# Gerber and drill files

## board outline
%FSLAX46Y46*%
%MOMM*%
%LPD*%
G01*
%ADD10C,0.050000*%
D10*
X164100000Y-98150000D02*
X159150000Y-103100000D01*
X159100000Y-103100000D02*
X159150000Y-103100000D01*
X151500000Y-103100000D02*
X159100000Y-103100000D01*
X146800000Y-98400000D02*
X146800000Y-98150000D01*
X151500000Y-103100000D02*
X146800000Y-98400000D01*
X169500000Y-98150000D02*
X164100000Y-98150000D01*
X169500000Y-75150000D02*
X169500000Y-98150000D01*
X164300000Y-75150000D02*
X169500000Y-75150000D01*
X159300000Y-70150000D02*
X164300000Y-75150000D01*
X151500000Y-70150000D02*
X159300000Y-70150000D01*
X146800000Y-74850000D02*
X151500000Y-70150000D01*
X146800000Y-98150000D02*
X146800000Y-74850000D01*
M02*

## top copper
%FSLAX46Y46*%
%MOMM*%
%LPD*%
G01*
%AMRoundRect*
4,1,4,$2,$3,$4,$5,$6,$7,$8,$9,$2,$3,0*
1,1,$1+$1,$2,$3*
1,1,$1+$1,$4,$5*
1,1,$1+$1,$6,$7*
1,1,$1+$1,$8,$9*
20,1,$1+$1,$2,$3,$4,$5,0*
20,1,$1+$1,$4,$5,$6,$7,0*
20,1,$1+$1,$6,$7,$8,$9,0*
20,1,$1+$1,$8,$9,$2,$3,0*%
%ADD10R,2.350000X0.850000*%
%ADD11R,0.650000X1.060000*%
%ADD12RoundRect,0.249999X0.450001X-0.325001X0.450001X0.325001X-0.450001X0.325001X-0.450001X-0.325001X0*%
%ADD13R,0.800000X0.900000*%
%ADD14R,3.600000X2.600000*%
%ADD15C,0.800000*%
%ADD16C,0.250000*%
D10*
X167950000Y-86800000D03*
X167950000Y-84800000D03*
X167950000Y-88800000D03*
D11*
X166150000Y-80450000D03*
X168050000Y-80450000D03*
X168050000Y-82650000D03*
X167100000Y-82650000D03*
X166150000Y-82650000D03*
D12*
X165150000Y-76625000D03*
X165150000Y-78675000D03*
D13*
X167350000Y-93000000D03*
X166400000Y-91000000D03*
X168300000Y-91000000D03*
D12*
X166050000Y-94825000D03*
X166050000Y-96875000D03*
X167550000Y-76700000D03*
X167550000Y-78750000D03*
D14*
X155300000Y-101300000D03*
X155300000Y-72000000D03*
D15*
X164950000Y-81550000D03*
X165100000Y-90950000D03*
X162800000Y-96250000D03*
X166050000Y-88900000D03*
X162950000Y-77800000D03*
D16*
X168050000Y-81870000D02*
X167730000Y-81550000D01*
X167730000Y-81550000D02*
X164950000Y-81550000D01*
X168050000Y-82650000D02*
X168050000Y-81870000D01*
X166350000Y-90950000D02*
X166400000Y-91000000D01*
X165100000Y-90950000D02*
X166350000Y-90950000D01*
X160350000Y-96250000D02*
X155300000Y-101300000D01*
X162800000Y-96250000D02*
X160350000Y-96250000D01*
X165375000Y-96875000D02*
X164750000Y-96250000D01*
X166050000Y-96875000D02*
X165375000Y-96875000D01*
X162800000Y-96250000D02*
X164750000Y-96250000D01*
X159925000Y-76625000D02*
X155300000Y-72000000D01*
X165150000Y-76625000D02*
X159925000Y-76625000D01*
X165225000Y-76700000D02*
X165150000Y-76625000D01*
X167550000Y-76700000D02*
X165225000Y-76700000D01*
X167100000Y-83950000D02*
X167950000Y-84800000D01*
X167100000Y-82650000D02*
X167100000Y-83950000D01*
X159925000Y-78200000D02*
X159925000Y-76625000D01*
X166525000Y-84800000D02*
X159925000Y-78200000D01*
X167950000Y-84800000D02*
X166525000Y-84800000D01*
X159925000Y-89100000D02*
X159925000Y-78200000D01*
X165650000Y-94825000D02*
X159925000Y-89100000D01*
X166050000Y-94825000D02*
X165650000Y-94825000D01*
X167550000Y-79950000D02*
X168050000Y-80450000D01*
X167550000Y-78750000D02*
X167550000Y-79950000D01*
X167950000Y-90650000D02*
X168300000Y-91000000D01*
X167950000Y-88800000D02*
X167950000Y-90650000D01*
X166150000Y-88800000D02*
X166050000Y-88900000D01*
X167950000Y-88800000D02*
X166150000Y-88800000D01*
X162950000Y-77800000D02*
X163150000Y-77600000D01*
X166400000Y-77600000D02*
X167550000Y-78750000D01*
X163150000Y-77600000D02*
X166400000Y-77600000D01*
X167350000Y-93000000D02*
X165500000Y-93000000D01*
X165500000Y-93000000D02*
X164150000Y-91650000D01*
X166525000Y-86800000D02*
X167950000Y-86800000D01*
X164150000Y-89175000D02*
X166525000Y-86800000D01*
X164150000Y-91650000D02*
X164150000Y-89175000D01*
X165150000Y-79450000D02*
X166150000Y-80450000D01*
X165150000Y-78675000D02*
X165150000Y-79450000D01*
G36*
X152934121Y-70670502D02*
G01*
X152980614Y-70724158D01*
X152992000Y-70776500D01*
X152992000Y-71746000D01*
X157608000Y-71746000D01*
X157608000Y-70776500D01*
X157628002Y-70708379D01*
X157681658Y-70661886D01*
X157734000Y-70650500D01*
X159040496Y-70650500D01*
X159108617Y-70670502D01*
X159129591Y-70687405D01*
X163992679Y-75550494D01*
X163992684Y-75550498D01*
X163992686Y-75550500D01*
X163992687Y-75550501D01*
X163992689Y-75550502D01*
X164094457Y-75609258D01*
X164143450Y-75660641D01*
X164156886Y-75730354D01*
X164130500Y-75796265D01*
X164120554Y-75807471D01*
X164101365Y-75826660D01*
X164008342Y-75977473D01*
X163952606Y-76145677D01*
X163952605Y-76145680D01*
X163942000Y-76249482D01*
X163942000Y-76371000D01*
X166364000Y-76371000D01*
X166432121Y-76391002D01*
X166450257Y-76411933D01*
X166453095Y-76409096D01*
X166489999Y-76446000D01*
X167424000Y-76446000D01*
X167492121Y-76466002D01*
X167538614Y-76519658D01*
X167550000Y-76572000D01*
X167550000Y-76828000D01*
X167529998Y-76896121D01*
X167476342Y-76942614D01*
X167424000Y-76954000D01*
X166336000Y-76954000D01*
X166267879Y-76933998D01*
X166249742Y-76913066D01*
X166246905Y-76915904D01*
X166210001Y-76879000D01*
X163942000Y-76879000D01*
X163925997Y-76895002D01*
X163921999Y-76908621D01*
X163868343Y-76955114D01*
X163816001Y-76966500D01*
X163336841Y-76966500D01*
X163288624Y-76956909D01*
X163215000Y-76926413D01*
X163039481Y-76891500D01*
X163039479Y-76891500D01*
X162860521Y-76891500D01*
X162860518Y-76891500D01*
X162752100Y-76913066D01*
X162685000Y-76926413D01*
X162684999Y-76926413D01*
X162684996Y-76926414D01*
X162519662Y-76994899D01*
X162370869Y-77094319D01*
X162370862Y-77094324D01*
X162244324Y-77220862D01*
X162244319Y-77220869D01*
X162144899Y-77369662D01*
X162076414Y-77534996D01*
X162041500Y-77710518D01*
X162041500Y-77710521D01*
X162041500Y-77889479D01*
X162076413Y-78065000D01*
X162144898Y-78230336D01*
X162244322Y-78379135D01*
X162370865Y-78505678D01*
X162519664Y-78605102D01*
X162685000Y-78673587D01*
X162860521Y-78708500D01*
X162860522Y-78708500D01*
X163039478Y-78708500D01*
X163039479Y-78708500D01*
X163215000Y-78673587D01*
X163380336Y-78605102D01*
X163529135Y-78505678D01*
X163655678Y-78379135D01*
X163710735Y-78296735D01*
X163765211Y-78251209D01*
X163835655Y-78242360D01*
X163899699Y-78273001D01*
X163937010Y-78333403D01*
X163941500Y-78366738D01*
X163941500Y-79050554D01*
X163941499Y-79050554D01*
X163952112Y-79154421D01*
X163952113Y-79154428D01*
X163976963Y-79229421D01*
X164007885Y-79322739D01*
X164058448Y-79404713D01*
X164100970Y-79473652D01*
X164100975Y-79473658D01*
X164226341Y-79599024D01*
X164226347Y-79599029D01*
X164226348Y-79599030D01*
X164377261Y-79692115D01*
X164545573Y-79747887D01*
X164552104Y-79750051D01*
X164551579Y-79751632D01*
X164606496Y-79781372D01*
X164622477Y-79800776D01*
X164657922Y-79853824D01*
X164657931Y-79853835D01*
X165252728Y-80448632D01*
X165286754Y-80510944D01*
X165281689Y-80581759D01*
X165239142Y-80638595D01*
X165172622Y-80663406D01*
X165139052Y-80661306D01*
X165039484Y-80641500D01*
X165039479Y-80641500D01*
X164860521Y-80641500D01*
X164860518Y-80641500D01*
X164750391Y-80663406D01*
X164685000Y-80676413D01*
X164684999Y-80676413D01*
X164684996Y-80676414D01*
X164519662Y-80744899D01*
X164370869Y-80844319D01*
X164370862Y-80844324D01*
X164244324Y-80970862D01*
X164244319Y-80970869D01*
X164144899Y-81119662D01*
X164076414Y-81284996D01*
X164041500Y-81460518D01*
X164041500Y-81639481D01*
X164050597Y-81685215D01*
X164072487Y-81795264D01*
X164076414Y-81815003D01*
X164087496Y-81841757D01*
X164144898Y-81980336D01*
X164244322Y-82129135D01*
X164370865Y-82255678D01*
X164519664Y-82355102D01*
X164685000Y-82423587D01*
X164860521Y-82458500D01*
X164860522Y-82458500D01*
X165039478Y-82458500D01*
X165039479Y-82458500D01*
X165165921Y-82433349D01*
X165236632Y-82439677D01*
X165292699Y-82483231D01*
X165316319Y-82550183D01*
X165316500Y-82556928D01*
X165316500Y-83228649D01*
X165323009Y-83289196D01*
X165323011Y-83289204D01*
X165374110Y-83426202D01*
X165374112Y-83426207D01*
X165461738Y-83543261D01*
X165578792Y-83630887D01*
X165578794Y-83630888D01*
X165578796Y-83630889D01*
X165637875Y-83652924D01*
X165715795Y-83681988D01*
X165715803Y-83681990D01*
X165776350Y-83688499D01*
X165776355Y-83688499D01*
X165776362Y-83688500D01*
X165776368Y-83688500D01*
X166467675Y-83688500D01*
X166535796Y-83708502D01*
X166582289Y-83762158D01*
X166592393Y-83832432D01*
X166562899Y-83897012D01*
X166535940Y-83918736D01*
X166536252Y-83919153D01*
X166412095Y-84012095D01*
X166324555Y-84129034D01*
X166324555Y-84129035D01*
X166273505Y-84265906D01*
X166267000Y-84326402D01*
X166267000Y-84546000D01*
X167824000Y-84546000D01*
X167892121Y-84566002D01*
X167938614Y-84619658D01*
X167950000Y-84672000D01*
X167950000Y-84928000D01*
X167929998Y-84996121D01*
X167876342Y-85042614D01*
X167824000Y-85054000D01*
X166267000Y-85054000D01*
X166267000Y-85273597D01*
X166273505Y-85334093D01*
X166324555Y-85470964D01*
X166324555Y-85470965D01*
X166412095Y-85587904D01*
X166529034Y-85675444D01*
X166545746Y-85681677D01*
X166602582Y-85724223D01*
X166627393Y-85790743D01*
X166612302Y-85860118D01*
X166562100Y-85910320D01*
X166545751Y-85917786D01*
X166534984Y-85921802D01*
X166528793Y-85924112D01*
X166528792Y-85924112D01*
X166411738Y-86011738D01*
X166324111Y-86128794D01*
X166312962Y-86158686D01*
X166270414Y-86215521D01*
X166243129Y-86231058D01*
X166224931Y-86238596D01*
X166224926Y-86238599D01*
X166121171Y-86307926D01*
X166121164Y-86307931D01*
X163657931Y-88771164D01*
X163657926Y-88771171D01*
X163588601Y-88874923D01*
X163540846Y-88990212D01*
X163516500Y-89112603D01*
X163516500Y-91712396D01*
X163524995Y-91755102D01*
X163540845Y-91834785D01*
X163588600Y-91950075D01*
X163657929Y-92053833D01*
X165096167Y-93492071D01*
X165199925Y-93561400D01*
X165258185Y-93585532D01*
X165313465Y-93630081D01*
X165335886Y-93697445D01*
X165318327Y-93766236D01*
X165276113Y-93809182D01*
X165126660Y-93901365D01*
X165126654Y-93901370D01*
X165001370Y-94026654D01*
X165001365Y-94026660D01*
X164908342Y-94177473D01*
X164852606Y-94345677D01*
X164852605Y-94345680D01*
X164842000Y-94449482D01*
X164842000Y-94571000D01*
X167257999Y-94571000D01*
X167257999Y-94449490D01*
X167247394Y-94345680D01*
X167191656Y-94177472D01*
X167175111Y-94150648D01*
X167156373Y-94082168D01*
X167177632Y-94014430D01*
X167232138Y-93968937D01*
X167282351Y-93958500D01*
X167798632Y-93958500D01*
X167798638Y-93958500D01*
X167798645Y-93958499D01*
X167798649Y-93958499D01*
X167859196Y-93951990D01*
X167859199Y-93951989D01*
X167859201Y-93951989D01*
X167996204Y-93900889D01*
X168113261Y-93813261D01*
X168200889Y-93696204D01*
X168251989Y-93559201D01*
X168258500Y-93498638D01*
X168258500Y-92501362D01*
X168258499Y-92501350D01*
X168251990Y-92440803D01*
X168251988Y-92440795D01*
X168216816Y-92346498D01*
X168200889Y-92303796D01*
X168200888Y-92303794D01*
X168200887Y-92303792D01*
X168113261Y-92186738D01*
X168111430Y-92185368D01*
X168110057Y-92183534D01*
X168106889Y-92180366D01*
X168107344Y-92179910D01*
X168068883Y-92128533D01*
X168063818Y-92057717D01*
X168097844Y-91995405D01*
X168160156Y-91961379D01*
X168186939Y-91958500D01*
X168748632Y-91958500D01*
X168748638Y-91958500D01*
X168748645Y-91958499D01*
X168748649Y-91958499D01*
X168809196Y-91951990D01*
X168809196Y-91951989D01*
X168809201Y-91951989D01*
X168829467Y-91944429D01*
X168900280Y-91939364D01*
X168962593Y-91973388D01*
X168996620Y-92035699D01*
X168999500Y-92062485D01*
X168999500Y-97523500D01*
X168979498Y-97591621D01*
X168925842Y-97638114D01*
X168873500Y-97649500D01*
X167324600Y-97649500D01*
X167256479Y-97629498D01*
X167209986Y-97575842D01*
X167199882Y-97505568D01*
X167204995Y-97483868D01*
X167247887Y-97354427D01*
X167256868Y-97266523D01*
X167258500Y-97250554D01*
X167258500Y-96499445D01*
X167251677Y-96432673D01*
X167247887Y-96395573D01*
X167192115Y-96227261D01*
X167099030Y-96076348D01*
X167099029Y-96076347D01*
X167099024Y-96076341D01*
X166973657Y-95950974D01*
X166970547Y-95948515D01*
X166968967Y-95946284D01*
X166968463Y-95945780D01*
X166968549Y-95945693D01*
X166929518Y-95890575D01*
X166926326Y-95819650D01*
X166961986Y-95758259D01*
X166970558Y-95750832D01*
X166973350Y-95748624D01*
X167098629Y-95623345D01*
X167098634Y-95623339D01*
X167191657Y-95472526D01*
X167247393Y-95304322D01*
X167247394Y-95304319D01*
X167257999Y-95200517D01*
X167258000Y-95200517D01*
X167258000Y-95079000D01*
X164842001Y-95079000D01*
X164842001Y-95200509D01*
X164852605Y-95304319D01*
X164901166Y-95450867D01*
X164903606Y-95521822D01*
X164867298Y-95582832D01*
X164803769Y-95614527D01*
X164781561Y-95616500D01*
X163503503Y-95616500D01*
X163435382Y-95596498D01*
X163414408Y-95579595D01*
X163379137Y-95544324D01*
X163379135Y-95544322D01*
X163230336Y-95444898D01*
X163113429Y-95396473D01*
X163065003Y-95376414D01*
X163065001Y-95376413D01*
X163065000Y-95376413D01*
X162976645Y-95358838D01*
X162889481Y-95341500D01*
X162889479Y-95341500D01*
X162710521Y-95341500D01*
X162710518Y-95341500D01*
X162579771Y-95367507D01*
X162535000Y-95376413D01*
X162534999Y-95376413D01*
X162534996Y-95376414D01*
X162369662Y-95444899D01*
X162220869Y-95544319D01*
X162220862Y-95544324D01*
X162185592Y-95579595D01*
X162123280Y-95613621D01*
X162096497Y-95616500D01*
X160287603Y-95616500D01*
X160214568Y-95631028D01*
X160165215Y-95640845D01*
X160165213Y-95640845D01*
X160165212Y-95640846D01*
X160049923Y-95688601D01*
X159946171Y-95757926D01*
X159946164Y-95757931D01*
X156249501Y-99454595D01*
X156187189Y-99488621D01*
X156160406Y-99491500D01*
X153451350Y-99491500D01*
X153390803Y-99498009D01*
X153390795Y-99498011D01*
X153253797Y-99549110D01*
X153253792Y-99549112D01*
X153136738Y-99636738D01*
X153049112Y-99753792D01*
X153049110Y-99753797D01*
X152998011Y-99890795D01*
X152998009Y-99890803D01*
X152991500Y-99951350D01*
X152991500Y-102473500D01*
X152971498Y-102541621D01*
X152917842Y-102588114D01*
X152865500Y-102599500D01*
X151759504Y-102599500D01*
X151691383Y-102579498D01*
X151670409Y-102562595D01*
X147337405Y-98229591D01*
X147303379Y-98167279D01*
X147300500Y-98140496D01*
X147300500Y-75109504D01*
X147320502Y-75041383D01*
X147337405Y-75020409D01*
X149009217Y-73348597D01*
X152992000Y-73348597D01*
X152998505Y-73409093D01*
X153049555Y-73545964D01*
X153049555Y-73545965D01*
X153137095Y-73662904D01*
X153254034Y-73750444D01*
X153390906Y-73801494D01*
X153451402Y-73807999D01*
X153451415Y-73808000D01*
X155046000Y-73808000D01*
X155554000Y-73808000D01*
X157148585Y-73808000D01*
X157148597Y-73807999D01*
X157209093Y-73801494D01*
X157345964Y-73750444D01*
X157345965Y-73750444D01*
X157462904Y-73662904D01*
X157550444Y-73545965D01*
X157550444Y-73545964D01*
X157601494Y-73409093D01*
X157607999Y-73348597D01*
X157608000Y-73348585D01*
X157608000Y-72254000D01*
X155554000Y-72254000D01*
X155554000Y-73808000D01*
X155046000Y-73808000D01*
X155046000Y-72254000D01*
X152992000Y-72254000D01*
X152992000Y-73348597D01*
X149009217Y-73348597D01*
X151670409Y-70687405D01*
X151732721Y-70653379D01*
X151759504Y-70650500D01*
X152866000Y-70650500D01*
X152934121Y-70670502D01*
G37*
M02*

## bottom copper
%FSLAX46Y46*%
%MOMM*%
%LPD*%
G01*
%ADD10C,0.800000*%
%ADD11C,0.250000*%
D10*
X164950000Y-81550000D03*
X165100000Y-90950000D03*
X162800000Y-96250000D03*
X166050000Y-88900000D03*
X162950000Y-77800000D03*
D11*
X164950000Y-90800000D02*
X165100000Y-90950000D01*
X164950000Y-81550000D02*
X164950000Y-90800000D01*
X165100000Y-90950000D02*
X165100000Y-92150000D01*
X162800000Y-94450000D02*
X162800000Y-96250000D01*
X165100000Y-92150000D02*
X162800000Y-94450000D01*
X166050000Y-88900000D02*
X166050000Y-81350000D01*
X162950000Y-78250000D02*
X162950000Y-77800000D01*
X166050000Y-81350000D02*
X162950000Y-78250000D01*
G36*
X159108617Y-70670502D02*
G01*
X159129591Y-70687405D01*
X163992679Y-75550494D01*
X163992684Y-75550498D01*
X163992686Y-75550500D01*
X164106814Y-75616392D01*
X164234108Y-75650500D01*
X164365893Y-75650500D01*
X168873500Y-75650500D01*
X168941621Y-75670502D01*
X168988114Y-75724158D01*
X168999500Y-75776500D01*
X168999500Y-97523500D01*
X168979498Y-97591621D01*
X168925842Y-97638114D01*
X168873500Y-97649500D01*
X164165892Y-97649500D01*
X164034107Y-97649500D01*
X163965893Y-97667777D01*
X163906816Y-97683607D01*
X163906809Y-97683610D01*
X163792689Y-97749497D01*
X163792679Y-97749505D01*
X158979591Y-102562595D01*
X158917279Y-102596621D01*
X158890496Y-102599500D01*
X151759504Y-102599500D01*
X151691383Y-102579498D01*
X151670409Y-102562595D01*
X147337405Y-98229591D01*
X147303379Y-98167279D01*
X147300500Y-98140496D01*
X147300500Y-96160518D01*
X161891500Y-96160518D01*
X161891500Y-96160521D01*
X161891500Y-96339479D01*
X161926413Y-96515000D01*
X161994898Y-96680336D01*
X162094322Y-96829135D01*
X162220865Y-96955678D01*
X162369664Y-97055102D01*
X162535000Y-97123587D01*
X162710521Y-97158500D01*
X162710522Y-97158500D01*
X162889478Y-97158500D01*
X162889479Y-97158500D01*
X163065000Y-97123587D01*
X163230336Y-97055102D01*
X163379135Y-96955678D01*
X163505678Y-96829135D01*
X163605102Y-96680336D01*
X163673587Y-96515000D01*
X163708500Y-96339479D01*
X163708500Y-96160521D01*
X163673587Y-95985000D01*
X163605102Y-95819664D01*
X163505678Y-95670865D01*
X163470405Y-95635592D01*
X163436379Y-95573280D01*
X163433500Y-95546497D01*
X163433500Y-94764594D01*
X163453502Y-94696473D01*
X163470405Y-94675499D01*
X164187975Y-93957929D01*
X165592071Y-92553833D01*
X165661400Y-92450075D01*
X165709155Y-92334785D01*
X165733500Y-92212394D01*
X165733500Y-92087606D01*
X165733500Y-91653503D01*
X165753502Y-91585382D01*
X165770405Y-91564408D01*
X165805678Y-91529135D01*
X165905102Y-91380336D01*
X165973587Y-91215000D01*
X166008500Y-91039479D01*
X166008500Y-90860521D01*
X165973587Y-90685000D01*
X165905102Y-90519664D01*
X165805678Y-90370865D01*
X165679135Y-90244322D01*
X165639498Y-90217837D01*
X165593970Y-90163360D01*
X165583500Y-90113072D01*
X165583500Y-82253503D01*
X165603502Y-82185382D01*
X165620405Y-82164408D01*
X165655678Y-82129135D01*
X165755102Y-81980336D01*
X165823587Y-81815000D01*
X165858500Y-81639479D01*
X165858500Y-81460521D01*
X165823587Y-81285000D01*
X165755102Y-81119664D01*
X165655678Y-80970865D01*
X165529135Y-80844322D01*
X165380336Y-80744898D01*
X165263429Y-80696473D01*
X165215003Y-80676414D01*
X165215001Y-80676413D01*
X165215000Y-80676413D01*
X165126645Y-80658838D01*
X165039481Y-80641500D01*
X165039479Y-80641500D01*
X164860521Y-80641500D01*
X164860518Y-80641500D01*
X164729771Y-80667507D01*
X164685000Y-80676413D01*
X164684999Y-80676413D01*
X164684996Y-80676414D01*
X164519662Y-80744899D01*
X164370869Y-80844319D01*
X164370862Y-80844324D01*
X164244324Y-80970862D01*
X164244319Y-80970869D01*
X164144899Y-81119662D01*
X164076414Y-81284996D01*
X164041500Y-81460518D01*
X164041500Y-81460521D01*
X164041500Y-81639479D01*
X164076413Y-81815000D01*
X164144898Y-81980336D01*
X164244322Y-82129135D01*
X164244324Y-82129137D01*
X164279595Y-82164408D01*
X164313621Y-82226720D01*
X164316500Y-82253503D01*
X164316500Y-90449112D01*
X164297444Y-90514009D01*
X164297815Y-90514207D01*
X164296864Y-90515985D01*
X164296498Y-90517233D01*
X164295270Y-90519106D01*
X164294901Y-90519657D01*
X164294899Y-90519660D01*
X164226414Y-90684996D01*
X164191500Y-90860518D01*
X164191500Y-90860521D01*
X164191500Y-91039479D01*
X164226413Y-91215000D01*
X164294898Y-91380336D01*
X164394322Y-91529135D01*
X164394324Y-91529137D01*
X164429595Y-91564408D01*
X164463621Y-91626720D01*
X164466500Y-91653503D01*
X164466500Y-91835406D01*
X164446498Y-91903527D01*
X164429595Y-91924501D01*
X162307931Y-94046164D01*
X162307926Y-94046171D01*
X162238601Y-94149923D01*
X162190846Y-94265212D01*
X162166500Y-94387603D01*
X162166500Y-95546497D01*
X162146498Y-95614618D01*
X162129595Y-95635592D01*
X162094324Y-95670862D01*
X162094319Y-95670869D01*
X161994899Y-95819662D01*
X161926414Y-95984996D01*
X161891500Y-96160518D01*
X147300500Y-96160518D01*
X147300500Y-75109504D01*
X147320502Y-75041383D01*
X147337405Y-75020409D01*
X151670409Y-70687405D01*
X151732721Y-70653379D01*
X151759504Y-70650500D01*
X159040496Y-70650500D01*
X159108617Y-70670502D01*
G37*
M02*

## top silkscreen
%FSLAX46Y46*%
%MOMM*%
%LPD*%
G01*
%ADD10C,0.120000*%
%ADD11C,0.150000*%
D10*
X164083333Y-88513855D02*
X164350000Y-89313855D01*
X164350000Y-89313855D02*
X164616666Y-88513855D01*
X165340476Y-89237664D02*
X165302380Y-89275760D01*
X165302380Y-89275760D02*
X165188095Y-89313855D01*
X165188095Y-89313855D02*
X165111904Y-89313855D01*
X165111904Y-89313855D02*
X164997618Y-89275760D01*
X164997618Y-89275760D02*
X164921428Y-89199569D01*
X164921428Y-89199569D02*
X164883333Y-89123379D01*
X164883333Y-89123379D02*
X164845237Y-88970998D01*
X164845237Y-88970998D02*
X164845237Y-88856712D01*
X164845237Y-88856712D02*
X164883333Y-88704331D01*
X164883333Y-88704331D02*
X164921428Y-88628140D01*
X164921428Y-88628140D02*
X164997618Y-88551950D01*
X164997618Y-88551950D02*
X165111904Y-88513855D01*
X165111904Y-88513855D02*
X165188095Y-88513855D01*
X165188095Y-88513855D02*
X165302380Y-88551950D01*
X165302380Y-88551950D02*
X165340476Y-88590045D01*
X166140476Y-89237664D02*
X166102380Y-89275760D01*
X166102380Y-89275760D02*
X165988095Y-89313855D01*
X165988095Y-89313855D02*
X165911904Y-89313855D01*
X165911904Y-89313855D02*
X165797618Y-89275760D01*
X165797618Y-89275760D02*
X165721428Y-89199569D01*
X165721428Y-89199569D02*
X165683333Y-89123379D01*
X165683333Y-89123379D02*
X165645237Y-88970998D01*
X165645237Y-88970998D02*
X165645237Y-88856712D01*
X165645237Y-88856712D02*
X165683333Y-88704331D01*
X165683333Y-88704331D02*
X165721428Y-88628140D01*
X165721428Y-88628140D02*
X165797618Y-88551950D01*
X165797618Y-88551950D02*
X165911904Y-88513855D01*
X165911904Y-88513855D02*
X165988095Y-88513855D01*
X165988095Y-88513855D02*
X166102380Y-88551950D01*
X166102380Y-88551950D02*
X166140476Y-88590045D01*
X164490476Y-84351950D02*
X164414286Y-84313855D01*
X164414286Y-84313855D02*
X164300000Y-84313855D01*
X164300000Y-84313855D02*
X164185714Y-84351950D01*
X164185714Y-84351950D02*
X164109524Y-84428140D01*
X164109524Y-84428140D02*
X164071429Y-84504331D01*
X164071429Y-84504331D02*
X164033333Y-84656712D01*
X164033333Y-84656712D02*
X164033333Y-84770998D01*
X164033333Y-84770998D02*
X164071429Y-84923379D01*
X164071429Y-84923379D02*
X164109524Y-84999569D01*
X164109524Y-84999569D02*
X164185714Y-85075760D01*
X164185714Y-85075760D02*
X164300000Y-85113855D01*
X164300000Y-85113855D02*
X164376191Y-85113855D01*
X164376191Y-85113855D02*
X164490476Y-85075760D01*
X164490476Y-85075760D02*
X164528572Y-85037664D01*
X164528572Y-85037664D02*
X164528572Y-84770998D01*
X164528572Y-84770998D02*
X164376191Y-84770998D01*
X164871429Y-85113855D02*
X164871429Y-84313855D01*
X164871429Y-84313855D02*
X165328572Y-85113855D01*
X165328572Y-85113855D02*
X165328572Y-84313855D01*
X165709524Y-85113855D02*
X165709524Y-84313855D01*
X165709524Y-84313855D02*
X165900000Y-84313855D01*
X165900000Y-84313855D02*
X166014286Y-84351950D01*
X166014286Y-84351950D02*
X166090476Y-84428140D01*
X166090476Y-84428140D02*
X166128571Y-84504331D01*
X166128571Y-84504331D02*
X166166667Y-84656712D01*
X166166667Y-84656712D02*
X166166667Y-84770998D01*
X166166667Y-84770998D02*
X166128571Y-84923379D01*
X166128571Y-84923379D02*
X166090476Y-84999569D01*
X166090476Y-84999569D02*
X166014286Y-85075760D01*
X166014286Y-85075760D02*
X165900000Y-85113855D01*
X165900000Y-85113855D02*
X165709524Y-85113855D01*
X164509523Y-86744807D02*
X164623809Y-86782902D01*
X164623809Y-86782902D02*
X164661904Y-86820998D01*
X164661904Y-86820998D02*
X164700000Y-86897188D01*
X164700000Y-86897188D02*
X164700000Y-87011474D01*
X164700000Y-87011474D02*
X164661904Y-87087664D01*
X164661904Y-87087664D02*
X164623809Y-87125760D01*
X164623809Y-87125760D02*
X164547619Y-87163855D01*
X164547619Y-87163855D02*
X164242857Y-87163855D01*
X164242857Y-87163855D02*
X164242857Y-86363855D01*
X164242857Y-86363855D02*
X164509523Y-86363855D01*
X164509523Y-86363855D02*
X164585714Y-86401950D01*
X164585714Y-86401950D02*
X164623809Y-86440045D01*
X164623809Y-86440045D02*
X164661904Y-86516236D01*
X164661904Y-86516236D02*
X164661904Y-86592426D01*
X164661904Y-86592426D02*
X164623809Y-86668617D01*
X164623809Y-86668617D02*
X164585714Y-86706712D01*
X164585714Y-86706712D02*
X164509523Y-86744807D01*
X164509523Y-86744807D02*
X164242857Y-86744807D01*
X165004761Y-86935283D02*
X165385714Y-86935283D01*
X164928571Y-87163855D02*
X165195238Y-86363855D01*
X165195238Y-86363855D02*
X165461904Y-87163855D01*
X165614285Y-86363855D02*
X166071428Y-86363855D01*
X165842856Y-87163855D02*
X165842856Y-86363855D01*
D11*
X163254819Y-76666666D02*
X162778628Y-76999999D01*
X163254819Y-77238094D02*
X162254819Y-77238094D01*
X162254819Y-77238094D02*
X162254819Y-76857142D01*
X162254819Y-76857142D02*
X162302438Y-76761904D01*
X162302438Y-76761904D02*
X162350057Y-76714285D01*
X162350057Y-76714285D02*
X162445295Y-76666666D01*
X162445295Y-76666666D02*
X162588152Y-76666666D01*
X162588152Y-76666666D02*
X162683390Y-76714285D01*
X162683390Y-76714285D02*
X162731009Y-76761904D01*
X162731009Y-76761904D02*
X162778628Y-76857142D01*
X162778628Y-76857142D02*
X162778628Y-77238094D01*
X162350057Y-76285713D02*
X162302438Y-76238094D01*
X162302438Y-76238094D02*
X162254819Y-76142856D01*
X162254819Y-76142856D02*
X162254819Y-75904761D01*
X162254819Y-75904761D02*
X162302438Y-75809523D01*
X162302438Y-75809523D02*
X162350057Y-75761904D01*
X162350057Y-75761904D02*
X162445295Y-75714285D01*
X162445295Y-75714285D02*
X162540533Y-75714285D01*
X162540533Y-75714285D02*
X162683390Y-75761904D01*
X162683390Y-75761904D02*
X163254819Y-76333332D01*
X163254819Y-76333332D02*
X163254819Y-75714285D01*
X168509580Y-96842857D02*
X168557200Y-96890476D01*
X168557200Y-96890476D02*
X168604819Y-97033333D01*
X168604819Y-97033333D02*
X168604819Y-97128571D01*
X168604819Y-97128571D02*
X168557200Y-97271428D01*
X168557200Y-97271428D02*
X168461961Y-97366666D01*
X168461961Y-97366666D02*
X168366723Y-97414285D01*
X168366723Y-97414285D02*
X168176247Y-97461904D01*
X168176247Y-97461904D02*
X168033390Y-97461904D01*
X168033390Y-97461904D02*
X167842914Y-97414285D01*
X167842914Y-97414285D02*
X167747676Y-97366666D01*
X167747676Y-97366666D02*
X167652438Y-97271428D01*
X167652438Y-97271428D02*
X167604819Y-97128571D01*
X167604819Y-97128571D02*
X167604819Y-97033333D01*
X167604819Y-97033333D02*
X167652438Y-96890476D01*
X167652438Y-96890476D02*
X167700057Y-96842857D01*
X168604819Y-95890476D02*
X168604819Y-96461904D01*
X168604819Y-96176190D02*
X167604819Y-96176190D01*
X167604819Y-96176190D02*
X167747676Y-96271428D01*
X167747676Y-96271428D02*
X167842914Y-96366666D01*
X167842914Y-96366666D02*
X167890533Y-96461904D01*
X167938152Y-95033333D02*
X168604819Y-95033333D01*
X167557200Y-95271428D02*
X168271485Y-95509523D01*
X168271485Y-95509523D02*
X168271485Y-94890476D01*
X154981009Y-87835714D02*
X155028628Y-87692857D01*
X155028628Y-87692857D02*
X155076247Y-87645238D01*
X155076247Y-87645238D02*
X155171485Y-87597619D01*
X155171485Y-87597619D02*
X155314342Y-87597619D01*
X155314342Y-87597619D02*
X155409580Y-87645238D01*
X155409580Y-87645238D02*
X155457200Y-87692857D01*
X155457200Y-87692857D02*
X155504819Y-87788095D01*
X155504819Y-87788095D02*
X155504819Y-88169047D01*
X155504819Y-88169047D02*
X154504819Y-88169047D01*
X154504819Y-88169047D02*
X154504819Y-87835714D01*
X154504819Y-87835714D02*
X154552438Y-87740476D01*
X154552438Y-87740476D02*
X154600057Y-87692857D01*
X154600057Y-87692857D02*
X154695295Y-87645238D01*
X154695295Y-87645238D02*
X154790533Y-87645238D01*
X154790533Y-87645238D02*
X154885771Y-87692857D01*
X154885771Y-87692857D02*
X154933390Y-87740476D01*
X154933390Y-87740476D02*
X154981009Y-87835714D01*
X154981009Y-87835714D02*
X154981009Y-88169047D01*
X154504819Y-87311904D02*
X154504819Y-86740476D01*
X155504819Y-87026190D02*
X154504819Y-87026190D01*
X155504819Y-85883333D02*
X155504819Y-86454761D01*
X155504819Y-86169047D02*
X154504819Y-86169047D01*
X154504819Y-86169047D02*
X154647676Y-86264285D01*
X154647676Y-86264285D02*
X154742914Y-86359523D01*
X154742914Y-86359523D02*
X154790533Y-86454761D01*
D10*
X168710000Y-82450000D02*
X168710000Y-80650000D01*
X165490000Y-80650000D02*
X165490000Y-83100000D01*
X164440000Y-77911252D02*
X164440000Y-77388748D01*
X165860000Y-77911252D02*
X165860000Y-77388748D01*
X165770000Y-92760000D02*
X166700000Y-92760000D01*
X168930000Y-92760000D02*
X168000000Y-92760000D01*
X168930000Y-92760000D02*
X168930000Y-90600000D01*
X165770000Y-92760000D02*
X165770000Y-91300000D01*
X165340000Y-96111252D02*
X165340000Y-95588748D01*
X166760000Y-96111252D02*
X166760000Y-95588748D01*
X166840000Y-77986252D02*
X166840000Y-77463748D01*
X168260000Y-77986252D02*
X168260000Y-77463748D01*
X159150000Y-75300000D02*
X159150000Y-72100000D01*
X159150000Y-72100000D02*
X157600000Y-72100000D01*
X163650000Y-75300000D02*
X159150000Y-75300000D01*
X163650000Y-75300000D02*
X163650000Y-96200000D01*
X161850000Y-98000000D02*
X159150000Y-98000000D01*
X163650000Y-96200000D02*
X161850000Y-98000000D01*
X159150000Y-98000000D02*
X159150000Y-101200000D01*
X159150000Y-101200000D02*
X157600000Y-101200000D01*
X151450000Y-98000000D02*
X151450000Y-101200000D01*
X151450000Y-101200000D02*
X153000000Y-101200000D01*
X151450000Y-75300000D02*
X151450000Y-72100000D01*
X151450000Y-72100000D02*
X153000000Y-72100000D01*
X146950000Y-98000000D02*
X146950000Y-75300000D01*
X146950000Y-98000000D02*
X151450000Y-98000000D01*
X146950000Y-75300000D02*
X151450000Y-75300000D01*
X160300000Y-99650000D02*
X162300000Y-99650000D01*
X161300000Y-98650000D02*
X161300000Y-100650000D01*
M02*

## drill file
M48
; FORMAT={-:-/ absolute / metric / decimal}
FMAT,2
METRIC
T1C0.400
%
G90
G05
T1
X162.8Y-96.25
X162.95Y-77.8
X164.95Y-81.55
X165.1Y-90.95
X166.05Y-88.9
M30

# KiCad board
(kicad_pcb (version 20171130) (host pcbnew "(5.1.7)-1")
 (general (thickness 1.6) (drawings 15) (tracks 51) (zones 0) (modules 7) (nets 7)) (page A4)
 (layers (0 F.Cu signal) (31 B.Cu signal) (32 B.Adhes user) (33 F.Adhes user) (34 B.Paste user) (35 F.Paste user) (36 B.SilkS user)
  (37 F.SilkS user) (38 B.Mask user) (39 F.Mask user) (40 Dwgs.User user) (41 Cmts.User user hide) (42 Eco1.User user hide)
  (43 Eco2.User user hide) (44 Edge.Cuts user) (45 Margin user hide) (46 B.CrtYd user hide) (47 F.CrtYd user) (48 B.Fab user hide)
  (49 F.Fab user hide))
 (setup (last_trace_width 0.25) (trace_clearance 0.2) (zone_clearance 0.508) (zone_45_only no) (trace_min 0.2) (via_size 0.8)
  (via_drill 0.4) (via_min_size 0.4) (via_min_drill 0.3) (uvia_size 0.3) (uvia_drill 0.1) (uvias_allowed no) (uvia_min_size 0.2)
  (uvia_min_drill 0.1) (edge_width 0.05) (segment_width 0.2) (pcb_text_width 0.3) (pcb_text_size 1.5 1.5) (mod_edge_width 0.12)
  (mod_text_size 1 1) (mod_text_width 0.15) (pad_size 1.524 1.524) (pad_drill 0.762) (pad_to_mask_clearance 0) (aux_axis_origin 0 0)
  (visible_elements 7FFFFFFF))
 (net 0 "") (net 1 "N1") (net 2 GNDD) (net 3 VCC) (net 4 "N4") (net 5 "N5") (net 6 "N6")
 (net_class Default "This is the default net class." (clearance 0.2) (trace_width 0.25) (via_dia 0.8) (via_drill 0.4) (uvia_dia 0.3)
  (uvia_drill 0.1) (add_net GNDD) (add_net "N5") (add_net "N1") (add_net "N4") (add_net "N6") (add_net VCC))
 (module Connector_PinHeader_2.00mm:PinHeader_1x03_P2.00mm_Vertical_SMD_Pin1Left (layer F.Cu) (at 167.95 86.8 180)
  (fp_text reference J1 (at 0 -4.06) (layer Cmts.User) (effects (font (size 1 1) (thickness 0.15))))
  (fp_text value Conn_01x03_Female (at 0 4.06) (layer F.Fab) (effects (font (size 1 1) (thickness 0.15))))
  (pad 2 smd rect (at 0 0 180) (size 2.35 0.85) (layers F.Cu F.Paste F.Mask) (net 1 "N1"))
  (pad 3 smd rect (at 0 2 180) (size 2.35 0.85) (layers F.Cu F.Paste F.Mask) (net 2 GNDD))
  (pad 1 smd rect (at 0 -2 180) (size 2.35 0.85) (layers F.Cu F.Paste F.Mask) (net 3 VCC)))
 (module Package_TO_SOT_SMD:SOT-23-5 (layer F.Cu) (at 167.1 81.55 90)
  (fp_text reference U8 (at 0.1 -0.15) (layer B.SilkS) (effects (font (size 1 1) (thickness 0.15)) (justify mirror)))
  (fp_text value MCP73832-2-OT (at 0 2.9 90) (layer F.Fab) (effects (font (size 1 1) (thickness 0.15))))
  (fp_line (start -0.9 1.61) (end 0.9 1.61) (layer F.SilkS) (width 0.12))
  (fp_line (start 0.9 -1.61) (end -1.55 -1.61) (layer F.SilkS) (width 0.12))
  (pad 5 smd rect (at 1.1 -0.95 90) (size 1.06 0.65) (layers F.Cu F.Paste F.Mask) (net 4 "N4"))
  (pad 4 smd rect (at 1.1 0.95 90) (size 1.06 0.65) (layers F.Cu F.Paste F.Mask) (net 3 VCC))
  (pad 3 smd rect (at -1.1 0.95 90) (size 1.06 0.65) (layers F.Cu F.Paste F.Mask) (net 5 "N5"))
  (pad 2 smd rect (at -1.1 0 90) (size 1.06 0.65) (layers F.Cu F.Paste F.Mask) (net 2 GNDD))
  (pad 1 smd rect (at -1.1 -0.95 90) (size 1.06 0.65) (layers F.Cu F.Paste F.Mask) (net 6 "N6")))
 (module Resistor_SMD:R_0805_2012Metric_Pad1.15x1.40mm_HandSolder (layer F.Cu) (at 165.15 77.65 90)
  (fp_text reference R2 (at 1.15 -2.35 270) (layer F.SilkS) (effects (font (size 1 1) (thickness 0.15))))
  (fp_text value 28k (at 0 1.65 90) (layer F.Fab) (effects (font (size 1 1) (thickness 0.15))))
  (fp_line (start -0.261252 -0.71) (end 0.261252 -0.71) (layer F.SilkS) (width 0.12))
  (fp_line (start -0.261252 0.71) (end 0.261252 0.71) (layer F.SilkS) (width 0.12))
  (pad 2 smd roundrect (at 1.025 0 90) (size 1.15 1.4) (layers F.Cu F.Paste F.Mask) (roundrect_rratio 0.2173904347826087) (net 2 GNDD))
  (pad 1 smd roundrect (at -1.025 0 90) (size 1.15 1.4) (layers F.Cu F.Paste F.Mask) (roundrect_rratio 0.2173904347826087) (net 4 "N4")))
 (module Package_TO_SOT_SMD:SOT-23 (layer F.Cu) (at 167.35 92 270)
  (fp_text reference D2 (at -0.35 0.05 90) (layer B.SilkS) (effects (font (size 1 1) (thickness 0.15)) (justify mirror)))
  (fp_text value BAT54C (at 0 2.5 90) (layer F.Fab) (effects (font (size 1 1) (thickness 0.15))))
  (fp_line (start 0.76 1.58) (end 0.76 0.65) (layer F.SilkS) (width 0.12))
  (fp_line (start 0.76 -1.58) (end 0.76 -0.65) (layer F.SilkS) (width 0.12))
  (fp_line (start 0.76 -1.58) (end -1.4 -1.58) (layer F.SilkS) (width 0.12))
  (fp_line (start 0.76 1.58) (end -0.7 1.58) (layer F.SilkS) (width 0.12))
  (pad 3 smd rect (at 1 0 270) (size 0.9 0.8) (layers F.Cu F.Paste F.Mask) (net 1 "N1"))
  (pad 2 smd rect (at -1 0.95 270) (size 0.9 0.8) (layers F.Cu F.Paste F.Mask) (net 5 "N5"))
  (pad 1 smd rect (at -1 -0.95 270) (size 0.9 0.8) (layers F.Cu F.Paste F.Mask) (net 3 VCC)))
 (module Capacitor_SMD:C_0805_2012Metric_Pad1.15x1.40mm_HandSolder (layer F.Cu) (at 166.05 95.85 90)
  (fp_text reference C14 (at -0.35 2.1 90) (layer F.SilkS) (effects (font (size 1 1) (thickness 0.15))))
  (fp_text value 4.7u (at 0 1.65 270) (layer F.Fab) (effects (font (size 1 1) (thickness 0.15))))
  (fp_line (start -0.261252 -0.71) (end 0.261252 -0.71) (layer F.SilkS) (width 0.12))
  (fp_line (start -0.261252 0.71) (end 0.261252 0.71) (layer F.SilkS) (width 0.12))
  (pad 2 smd roundrect (at 1.025 0 90) (size 1.15 1.4) (layers F.Cu F.Paste F.Mask) (roundrect_rratio 0.2173904347826087) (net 2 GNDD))
  (pad 1 smd roundrect (at -1.025 0 90) (size 1.15 1.4) (layers F.Cu F.Paste F.Mask) (roundrect_rratio 0.2173904347826087) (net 5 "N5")))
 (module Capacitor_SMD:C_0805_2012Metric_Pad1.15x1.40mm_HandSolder (layer F.Cu) (at 167.55 77.725 90)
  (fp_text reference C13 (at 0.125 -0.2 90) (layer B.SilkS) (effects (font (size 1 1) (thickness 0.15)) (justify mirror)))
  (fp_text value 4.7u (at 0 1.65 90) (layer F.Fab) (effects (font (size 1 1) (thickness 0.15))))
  (fp_line (start -0.261252 -0.71) (end 0.261252 -0.71) (layer F.SilkS) (width 0.12))
  (fp_line (start -0.261252 0.71) (end 0.261252 0.71) (layer F.SilkS) (width 0.12))
  (pad 2 smd roundrect (at 1.025 0 90) (size 1.15 1.4) (layers F.Cu F.Paste F.Mask) (roundrect_rratio 0.2173904347826087) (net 2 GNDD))
  (pad 1 smd roundrect (at -1.025 0 90) (size 1.15 1.4) (layers F.Cu F.Paste F.Mask) (roundrect_rratio 0.2173904347826087) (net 3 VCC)))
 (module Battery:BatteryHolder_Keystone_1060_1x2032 (layer F.Cu) (at 155.3 86.65 90)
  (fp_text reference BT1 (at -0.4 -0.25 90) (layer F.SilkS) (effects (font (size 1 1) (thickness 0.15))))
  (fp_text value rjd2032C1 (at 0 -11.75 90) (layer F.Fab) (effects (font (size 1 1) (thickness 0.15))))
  (fp_line (start 11.35 3.85) (end 14.55 3.85) (layer F.SilkS) (width 0.12))
  (fp_line (start 14.55 3.85) (end 14.55 2.3) (layer F.SilkS) (width 0.12))
  (fp_line (start 11.35 8.35) (end 11.35 3.85) (layer F.SilkS) (width 0.12))
  (fp_line (start 11.35 8.35) (end -9.55 8.35) (layer F.SilkS) (width 0.12))
  (fp_line (start -11.35 6.55) (end -11.35 3.85) (layer F.SilkS) (width 0.12))
  (fp_line (start -9.55 8.35) (end -11.35 6.55) (layer F.SilkS) (width 0.12))
  (fp_line (start -11.35 3.85) (end -14.55 3.85) (layer F.SilkS) (width 0.12))
  (fp_line (start -14.55 3.85) (end -14.55 2.3) (layer F.SilkS) (width 0.12))
  (fp_line (start -11.35 -3.85) (end -14.55 -3.85) (layer F.SilkS) (width 0.12))
  (fp_line (start -14.55 -3.85) (end -14.55 -2.3) (layer F.SilkS) (width 0.12))
  (fp_line (start 11.35 -3.85) (end 14.55 -3.85) (layer F.SilkS) (width 0.12))
  (fp_line (start 14.55 -3.85) (end 14.55 -2.3) (layer F.SilkS) (width 0.12))
  (fp_line (start -11.35 -8.35) (end 11.35 -8.35) (layer F.SilkS) (width 0.12))
  (fp_line (start -11.35 -8.35) (end -11.35 -3.85) (layer F.SilkS) (width 0.12))
  (fp_line (start 11.35 -8.35) (end 11.35 -3.85) (layer F.SilkS) (width 0.12))
  (fp_line (start -13 5) (end -13 7) (layer F.SilkS) (width 0.12))
  (fp_line (start -12 6) (end -14 6) (layer F.SilkS) (width 0.12))
  (pad 1 smd rect (at -14.65 0 270) (size 2.6 3.6) (layers F.Cu F.Paste F.Mask) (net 5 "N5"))
  (pad 2 smd rect (at 14.65 0 270) (size 2.6 3.6) (layers F.Cu F.Paste F.Mask) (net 2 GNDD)))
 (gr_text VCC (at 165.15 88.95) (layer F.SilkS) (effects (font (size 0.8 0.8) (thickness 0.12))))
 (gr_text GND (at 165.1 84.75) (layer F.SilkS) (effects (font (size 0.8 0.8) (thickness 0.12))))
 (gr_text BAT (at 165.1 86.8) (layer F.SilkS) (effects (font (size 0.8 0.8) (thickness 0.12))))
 (gr_line (start 164.1 98.15) (end 159.15 103.1) (layer Edge.Cuts) (width 0.05))
 (gr_line (start 159.1 103.1) (end 159.15 103.1) (layer Edge.Cuts) (width 0.05))
 (gr_line (start 151.5 103.1) (end 159.1 103.1) (layer Edge.Cuts) (width 0.05))
 (gr_line (start 146.8 98.4) (end 146.8 98.15) (layer Edge.Cuts) (width 0.05))
 (gr_line (start 151.5 103.1) (end 146.8 98.4) (layer Edge.Cuts) (width 0.05))
 (gr_line (start 169.5 98.15) (end 164.1 98.15) (layer Edge.Cuts) (width 0.05))
 (gr_line (start 169.5 75.15) (end 169.5 98.15) (layer Edge.Cuts) (width 0.05))
 (gr_line (start 164.3 75.15) (end 169.5 75.15) (layer Edge.Cuts) (width 0.05))
 (gr_line (start 159.3 70.15) (end 164.3 75.15) (layer Edge.Cuts) (width 0.05))
 (gr_line (start 151.5 70.15) (end 159.3 70.15) (layer Edge.Cuts) (width 0.05))
 (gr_line (start 146.8 74.85) (end 151.5 70.15) (layer Edge.Cuts) (width 0.05))
 (gr_line (start 146.8 98.15) (end 146.8 74.85) (layer Edge.Cuts) (width 0.05))
 (via (at 164.95 81.55) (size 0.8) (drill 0.4) (layers F.Cu B.Cu) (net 5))
 (segment (start 168.05 81.87) (end 167.73 81.55) (width 0.25) (layer F.Cu) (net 5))
 (segment (start 167.73 81.55) (end 164.95 81.55) (width 0.25) (layer F.Cu) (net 5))
 (segment (start 168.05 82.65) (end 168.05 81.87) (width 0.25) (layer F.Cu) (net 5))
 (segment (start 164.95 90.8) (end 165.1 90.95) (width 0.25) (layer B.Cu) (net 5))
 (via (at 165.1 90.95) (size 0.8) (drill 0.4) (layers F.Cu B.Cu) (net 5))
 (segment (start 164.95 81.55) (end 164.95 90.8) (width 0.25) (layer B.Cu) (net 5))
 (segment (start 166.35 90.95) (end 166.4 91) (width 0.25) (layer F.Cu) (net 5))
 (segment (start 165.1 90.95) (end 166.35 90.95) (width 0.25) (layer F.Cu) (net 5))
 (segment (start 165.1 90.95) (end 165.1 92.15) (width 0.25) (layer B.Cu) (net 5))
 (via (at 162.8 96.25) (size 0.8) (drill 0.4) (layers F.Cu B.Cu) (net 5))
 (segment (start 162.8 94.45) (end 162.8 96.25) (width 0.25) (layer B.Cu) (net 5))
 (segment (start 165.1 92.15) (end 162.8 94.45) (width 0.25) (layer B.Cu) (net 5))
 (segment (start 160.35 96.25) (end 155.3 101.3) (width 0.25) (layer F.Cu) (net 5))
 (segment (start 162.8 96.25) (end 160.35 96.25) (width 0.25) (layer F.Cu) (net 5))
 (segment (start 165.375 96.875) (end 164.75 96.25) (width 0.25) (layer F.Cu) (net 5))
 (segment (start 166.05 96.875) (end 165.375 96.875) (width 0.25) (layer F.Cu) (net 5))
 (segment (start 162.8 96.25) (end 164.75 96.25) (width 0.25) (layer F.Cu) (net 5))
 (segment (start 159.925 76.625) (end 155.3 72) (width 0.25) (layer F.Cu) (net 2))
 (segment (start 165.15 76.625) (end 159.925 76.625) (width 0.25) (layer F.Cu) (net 2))
 (segment (start 165.225 76.7) (end 165.15 76.625) (width 0.25) (layer F.Cu) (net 2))
 (segment (start 167.55 76.7) (end 165.225 76.7) (width 0.25) (layer F.Cu) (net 2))
 (segment (start 167.1 83.95) (end 167.95 84.8) (width 0.25) (layer F.Cu) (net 2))
 (segment (start 167.1 82.65) (end 167.1 83.95) (width 0.25) (layer F.Cu) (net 2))
 (segment (start 159.925 78.2) (end 159.925 76.625) (width 0.25) (layer F.Cu) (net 2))
 (segment (start 166.525 84.8) (end 159.925 78.2) (width 0.25) (layer F.Cu) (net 2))
 (segment (start 167.95 84.8) (end 166.525 84.8) (width 0.25) (layer F.Cu) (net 2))
 (segment (start 159.925 89.1) (end 159.925 78.2) (width 0.25) (layer F.Cu) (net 2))
 (segment (start 165.65 94.825) (end 159.925 89.1) (width 0.25) (layer F.Cu) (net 2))
 (segment (start 166.05 94.825) (end 165.65 94.825) (width 0.25) (layer F.Cu) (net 2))
 (segment (start 167.55 79.95) (end 168.05 80.45) (width 0.25) (layer F.Cu) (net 3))
 (segment (start 167.55 78.75) (end 167.55 79.95) (width 0.25) (layer F.Cu) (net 3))
 (segment (start 167.95 90.65) (end 168.3 91) (width 0.25) (layer F.Cu) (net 3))
 (segment (start 167.95 88.8) (end 167.95 90.65) (width 0.25) (layer F.Cu) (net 3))
 (via (at 166.05 88.9) (size 0.8) (drill 0.4) (layers F.Cu B.Cu) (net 3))
 (segment (start 166.15 88.8) (end 166.05 88.9) (width 0.25) (layer F.Cu) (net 3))
 (segment (start 167.95 88.8) (end 166.15 88.8) (width 0.25) (layer F.Cu) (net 3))
 (segment (start 166.05 88.9) (end 166.05 81.35) (width 0.25) (layer B.Cu) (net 3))
 (via (at 162.95 77.8) (size 0.8) (drill 0.4) (layers F.Cu B.Cu) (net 3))
 (segment (start 162.95 78.25) (end 162.95 77.8) (width 0.25) (layer B.Cu) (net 3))
 (segment (start 166.05 81.35) (end 162.95 78.25) (width 0.25) (layer B.Cu) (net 3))
 (segment (start 162.95 77.8) (end 163.15 77.6) (width 0.25) (layer F.Cu) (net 3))
 (segment (start 166.4 77.6) (end 167.55 78.75) (width 0.25) (layer F.Cu) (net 3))
 (segment (start 163.15 77.6) (end 166.4 77.6) (width 0.25) (layer F.Cu) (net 3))
 (segment (start 167.35 93) (end 165.5 93) (width 0.25) (layer F.Cu) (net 1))
 (segment (start 165.5 93) (end 164.15 91.65) (width 0.25) (layer F.Cu) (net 1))
 (segment (start 166.525 86.8) (end 167.95 86.8) (width 0.25) (layer F.Cu) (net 1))
 (segment (start 164.15 89.175) (end 166.525 86.8) (width 0.25) (layer F.Cu) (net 1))
 (segment (start 164.15 91.65) (end 164.15 89.175) (width 0.25) (layer F.Cu) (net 1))
 (segment (start 165.15 79.45) (end 166.15 80.45) (width 0.25) (layer F.Cu) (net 4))
 (segment (start 165.15 78.675) (end 165.15 79.45) (width 0.25) (layer F.Cu) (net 4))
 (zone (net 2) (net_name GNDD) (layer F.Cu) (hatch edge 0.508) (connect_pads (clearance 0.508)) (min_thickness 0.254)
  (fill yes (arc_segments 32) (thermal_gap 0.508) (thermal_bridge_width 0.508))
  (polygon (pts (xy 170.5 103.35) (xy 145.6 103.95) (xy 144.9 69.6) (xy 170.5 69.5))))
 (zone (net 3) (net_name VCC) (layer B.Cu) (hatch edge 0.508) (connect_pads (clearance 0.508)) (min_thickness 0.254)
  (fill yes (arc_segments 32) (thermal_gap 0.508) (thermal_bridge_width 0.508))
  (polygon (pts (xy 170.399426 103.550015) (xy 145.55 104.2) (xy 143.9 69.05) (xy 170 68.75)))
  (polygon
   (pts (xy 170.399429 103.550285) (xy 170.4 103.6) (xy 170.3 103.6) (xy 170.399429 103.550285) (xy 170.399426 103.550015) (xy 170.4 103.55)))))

